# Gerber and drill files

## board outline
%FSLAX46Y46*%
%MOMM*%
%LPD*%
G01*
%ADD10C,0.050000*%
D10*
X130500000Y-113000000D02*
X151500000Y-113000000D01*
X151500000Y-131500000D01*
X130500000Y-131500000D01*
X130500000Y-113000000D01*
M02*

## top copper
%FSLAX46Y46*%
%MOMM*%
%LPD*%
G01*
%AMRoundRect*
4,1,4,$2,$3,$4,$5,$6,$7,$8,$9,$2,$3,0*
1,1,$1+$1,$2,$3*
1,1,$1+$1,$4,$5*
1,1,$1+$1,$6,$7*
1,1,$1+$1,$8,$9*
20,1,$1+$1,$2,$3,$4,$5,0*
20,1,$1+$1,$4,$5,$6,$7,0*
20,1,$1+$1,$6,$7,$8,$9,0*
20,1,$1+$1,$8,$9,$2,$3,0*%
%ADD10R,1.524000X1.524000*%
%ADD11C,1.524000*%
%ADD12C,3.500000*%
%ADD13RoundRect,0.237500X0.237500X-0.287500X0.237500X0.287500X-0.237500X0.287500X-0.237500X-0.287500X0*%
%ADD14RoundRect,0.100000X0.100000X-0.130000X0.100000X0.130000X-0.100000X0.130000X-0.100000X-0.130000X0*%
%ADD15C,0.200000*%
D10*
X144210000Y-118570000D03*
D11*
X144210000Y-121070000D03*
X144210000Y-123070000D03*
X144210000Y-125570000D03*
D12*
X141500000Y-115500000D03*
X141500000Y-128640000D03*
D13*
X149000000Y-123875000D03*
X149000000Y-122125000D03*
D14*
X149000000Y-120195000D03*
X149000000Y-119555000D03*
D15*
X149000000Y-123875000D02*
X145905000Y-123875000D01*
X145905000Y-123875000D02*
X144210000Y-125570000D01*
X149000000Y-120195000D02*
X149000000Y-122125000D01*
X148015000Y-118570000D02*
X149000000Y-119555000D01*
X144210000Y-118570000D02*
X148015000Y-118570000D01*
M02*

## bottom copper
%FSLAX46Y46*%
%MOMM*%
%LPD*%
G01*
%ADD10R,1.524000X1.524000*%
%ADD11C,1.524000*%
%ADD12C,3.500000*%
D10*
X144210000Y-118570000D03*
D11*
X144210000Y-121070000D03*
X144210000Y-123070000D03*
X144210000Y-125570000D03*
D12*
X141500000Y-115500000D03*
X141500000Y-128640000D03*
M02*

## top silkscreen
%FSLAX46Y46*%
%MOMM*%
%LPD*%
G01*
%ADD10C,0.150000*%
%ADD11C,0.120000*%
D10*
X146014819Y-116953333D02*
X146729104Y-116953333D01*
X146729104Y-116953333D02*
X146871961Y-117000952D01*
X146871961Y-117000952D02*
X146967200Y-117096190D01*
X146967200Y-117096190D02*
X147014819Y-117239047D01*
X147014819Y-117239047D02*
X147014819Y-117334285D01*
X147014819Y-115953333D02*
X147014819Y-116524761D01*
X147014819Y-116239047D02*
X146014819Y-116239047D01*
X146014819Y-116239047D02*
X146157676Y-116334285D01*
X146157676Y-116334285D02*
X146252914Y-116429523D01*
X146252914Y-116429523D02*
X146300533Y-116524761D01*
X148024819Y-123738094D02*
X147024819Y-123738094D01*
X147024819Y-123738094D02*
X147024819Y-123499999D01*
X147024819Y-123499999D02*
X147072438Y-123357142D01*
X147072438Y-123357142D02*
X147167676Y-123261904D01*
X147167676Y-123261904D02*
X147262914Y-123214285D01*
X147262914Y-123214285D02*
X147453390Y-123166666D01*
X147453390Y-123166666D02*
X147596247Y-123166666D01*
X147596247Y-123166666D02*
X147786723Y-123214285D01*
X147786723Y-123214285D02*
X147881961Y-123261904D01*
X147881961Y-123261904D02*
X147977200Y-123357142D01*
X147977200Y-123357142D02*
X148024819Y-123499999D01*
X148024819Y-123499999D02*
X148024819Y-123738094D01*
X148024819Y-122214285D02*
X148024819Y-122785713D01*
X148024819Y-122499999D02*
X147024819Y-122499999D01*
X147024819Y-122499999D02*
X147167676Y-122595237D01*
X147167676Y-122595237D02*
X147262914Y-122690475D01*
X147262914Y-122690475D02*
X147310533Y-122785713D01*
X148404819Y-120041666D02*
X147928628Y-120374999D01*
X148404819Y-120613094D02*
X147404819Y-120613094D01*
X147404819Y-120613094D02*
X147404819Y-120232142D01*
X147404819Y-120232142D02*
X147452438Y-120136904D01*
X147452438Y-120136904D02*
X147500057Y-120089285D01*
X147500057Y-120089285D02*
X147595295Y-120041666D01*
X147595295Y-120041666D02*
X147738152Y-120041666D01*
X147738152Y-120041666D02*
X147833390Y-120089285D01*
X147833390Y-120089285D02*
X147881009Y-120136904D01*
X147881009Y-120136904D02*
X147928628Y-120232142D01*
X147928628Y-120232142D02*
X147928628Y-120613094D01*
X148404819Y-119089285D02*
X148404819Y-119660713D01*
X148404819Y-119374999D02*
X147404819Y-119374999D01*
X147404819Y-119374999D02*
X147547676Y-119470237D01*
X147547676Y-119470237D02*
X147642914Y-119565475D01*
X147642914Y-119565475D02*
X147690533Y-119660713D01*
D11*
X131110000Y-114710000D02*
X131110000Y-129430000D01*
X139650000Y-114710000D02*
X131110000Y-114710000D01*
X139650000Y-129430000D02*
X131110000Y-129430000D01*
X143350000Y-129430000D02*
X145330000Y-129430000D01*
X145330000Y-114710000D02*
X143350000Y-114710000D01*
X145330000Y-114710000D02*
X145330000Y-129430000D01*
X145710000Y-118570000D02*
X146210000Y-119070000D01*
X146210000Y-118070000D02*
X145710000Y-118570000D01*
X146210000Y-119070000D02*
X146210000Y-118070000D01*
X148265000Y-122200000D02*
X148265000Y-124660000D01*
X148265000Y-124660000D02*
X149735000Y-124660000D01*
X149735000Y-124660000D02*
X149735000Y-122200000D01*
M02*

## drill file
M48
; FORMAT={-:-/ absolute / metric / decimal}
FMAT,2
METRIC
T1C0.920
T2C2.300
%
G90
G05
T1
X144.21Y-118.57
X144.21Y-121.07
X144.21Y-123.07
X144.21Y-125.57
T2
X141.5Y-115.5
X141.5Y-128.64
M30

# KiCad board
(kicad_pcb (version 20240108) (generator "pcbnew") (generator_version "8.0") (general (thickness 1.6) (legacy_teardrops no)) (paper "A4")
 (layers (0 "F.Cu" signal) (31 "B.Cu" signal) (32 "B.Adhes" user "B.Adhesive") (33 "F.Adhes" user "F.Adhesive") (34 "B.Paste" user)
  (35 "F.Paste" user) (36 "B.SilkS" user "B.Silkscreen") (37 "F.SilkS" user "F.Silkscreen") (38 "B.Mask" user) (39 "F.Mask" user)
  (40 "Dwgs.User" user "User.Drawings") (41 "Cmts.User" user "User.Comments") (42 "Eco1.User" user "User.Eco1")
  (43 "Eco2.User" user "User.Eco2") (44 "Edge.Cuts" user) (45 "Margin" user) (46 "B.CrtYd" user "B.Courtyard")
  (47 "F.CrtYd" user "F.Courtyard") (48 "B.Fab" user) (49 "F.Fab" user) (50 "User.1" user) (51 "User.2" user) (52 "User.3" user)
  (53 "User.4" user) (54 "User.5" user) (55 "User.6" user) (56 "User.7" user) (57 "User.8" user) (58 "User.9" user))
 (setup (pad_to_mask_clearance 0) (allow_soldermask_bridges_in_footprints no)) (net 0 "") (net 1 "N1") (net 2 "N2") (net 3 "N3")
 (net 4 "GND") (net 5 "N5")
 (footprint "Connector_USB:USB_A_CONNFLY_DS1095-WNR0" (layer "F.Cu") (at 144.21 118.57 -90)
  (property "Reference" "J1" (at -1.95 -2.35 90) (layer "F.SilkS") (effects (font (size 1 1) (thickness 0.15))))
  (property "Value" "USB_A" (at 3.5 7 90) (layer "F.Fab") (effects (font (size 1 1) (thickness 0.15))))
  (fp_line (start -3.86 13.1) (end 10.86 13.1) (stroke (width 0.12) (type solid)) (layer "F.SilkS"))
  (fp_line (start -3.86 4.56) (end -3.86 13.1) (stroke (width 0.12) (type solid)) (layer "F.SilkS"))
  (fp_line (start 10.86 4.56) (end 10.86 13.1) (stroke (width 0.12) (type solid)) (layer "F.SilkS"))
  (fp_line (start 10.86 0.86) (end 10.86 -1.12) (stroke (width 0.12) (type solid)) (layer "F.SilkS"))
  (fp_line (start -3.86 -1.12) (end -3.86 0.86) (stroke (width 0.12) (type solid)) (layer "F.SilkS"))
  (fp_line (start -3.86 -1.12) (end 10.86 -1.12) (stroke (width 0.12) (type solid)) (layer "F.SilkS"))
  (fp_line (start 0 -1.5) (end 0.5 -2) (stroke (width 0.12) (type solid)) (layer "F.SilkS"))
  (fp_line (start -0.5 -2) (end 0 -1.5) (stroke (width 0.12) (type solid)) (layer "F.SilkS"))
  (fp_line (start 0.5 -2) (end -0.5 -2) (stroke (width 0.12) (type solid)) (layer "F.SilkS"))
  (pad "1" thru_hole rect (at 0 0 270) (size 1.524 1.524) (drill 0.92) (layers "*.Cu" "*.Mask") (remove_unused_layers no) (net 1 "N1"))
  (pad "2" thru_hole circle (at 2.5 0 270) (size 1.524 1.524) (drill 0.92) (layers "*.Cu" "*.Mask") (remove_unused_layers no) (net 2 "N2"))
  (pad "3" thru_hole circle (at 4.5 0 270) (size 1.524 1.524) (drill 0.92) (layers "*.Cu" "*.Mask") (remove_unused_layers no) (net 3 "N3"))
  (pad "4" thru_hole circle (at 7 0 270) (size 1.524 1.524) (drill 0.92) (layers "*.Cu" "*.Mask") (remove_unused_layers no) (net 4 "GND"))
  (pad "5" thru_hole circle (at -3.07 2.71 270) (size 3.5 3.5) (drill 2.3) (layers "*.Cu" "*.Mask") (remove_unused_layers no) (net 4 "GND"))
  (pad "5" thru_hole circle (at 10.07 2.71 270) (size 3.5 3.5) (drill 2.3) (layers "*.Cu" "*.Mask") (remove_unused_layers no) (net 4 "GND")))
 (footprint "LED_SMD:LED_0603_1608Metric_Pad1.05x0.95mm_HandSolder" (layer "F.Cu") (at 149 123 90)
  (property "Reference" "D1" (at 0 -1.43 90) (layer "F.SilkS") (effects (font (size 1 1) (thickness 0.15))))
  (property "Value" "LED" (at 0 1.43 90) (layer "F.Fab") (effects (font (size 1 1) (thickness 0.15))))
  (fp_line (start 0.8 -0.735) (end -1.66 -0.735) (stroke (width 0.12) (type solid)) (layer "F.SilkS"))
  (fp_line (start -1.66 -0.735) (end -1.66 0.735) (stroke (width 0.12) (type solid)) (layer "F.SilkS"))
  (fp_line (start -1.66 0.735) (end 0.8 0.735) (stroke (width 0.12) (type solid)) (layer "F.SilkS"))
  (pad "1" smd roundrect (at -0.875 0 90) (size 1.05 0.95) (layers "F.Cu" "F.Paste" "F.Mask") (roundrect_rratio 0.25) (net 4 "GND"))
  (pad "2" smd roundrect (at 0.875 0 90) (size 1.05 0.95) (layers "F.Cu" "F.Paste" "F.Mask") (roundrect_rratio 0.25) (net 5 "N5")))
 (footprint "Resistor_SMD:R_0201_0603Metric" (layer "F.Cu") (at 149 119.875 90)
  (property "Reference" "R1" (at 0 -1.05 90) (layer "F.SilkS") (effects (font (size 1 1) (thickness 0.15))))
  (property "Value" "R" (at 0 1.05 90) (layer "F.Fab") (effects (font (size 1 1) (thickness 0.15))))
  (pad "" smd roundrect (at -0.345 0 90) (size 0.318 0.36) (layers "F.Paste") (roundrect_rratio 0.25))
  (pad "" smd roundrect (at 0.345 0 90) (size 0.318 0.36) (layers "F.Paste") (roundrect_rratio 0.25))
  (pad "1" smd roundrect (at -0.32 0 90) (size 0.46 0.4) (layers "F.Cu" "F.Mask") (roundrect_rratio 0.25) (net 5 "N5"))
  (pad "2" smd roundrect (at 0.32 0 90) (size 0.46 0.4) (layers "F.Cu" "F.Mask") (roundrect_rratio 0.25) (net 1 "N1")))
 (gr_rect (start 130.5 113) (end 151.5 131.5) (stroke (width 0.05) (type default)) (fill none) (layer "Edge.Cuts"))
 (segment (start 149 123.875) (end 145.905 123.875) (width 0.2) (layer "F.Cu") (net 4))
 (segment (start 145.905 123.875) (end 144.21 125.57) (width 0.2) (layer "F.Cu") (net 4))
 (segment (start 149 120.195) (end 149 122.125) (width 0.2) (layer "F.Cu") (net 5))
 (segment (start 148.015 118.57) (end 149 119.555) (width 0.2) (layer "F.Cu") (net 1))
 (segment (start 144.21 118.57) (end 148.015 118.57) (width 0.2) (layer "F.Cu") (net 1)))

